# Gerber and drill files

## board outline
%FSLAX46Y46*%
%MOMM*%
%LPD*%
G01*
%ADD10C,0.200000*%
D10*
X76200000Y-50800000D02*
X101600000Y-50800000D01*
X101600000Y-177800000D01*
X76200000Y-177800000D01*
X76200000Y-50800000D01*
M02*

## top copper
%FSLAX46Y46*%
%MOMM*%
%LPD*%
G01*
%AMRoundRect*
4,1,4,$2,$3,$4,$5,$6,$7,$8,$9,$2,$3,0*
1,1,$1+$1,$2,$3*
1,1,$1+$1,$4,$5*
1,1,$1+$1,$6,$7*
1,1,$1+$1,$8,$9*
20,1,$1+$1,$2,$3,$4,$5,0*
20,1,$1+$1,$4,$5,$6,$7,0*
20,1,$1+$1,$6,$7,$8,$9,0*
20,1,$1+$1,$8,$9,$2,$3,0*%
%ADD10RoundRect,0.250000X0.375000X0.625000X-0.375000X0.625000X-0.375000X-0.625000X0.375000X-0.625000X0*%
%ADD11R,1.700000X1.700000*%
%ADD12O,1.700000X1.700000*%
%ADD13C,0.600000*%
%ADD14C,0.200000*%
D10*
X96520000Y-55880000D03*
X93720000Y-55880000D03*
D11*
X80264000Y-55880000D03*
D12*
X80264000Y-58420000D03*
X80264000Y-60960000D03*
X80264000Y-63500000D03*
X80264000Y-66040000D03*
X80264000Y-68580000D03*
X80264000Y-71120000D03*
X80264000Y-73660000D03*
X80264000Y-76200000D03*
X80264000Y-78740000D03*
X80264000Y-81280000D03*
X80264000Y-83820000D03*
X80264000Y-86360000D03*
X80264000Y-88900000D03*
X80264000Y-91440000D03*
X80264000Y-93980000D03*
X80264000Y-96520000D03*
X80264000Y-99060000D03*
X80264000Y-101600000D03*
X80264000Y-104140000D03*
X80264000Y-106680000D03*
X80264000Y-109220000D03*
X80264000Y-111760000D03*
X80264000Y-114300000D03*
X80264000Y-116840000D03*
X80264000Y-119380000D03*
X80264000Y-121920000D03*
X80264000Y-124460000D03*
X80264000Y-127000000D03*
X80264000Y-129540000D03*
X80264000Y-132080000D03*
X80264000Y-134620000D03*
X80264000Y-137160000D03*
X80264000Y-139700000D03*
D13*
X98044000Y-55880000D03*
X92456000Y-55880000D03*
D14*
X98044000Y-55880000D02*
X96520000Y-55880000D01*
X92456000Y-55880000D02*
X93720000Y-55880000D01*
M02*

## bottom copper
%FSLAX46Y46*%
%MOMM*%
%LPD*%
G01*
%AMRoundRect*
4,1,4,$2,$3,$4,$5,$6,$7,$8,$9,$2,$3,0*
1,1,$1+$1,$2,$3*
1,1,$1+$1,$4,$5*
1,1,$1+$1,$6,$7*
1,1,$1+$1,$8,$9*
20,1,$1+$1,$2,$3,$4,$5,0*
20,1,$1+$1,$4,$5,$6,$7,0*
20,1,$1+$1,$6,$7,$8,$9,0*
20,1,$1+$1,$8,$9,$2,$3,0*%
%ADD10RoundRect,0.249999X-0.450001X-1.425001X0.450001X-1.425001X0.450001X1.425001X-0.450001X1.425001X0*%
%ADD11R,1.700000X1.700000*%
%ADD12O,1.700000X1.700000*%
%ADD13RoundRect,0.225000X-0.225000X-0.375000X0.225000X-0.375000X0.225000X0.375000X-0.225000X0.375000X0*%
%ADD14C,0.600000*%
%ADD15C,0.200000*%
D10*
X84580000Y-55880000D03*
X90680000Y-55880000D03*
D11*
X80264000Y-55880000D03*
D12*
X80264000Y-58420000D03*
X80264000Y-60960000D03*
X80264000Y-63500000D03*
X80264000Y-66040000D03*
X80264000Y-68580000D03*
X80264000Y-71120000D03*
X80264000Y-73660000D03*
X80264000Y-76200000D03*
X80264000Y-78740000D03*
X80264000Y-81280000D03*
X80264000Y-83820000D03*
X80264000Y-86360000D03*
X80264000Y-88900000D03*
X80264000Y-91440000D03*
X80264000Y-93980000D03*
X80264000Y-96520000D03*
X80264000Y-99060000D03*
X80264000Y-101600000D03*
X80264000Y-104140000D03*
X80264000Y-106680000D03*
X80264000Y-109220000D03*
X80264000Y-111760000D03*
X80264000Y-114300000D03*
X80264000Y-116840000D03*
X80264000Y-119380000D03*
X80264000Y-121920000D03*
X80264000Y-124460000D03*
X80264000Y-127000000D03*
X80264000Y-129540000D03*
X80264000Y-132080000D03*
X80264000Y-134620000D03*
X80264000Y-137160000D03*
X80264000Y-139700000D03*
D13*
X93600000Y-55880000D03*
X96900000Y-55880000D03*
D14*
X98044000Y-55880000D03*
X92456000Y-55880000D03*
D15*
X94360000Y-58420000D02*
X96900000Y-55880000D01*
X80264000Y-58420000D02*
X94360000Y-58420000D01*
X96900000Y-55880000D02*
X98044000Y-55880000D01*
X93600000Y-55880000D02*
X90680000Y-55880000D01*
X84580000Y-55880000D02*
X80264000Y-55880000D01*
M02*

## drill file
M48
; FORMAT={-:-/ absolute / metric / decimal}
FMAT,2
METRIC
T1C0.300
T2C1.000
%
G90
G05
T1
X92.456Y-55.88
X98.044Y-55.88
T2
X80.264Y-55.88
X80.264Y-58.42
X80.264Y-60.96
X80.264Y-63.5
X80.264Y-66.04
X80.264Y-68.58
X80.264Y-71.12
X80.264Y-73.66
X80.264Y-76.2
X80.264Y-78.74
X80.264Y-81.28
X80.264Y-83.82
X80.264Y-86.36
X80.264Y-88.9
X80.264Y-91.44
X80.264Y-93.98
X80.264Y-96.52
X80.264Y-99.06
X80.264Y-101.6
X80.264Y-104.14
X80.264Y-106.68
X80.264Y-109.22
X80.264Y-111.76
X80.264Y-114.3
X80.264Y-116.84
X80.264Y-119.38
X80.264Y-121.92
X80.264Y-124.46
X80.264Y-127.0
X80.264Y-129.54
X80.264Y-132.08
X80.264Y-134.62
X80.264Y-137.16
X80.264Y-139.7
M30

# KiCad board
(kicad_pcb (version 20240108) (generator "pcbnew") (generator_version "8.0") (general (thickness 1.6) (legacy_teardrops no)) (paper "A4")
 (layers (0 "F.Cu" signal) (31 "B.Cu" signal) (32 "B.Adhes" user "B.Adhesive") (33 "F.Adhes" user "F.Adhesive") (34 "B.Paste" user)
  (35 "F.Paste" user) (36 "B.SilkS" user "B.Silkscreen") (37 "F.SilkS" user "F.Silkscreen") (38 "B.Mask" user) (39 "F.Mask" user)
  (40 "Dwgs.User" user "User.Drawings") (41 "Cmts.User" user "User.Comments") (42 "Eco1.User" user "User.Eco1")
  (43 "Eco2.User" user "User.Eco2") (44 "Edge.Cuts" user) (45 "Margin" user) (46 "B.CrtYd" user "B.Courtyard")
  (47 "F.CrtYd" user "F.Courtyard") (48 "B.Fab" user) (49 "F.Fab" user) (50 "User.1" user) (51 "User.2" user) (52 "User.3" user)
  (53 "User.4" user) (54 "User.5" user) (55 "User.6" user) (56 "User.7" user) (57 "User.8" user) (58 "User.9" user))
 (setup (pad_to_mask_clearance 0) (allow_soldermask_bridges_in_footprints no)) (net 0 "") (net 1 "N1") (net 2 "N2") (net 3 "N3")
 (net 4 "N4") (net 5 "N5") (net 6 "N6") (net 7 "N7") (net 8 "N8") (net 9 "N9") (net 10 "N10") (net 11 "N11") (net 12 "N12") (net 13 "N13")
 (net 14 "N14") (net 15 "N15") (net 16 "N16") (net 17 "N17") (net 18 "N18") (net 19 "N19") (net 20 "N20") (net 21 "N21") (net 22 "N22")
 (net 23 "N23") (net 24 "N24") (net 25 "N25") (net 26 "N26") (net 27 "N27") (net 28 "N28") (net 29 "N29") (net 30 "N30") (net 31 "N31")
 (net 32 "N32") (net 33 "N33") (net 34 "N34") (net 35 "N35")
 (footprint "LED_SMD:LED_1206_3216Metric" (layer "F.Cu") (at 95.12 55.88 180)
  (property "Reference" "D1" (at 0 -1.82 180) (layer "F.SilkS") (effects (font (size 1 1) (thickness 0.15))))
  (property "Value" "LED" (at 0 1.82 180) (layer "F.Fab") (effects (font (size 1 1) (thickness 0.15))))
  (pad "1" smd roundrect (at -1.4 0 180) (size 1.25 1.75) (layers "F.Cu" "F.Paste" "F.Mask") (roundrect_rratio 0.2) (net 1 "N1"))
  (pad "2" smd roundrect (at 1.4 0 180) (size 1.25 1.75) (layers "F.Cu" "F.Paste" "F.Mask") (roundrect_rratio 0.2) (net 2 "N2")))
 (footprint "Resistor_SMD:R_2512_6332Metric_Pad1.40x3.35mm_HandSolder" (layer "B.Cu") (at 87.63 55.88)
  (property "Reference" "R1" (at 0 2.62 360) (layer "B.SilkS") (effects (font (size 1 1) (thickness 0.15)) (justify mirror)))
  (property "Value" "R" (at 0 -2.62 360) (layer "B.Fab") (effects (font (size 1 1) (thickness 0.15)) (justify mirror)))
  (pad "1" smd roundrect (at -3.05 0) (size 1.4 3.35) (layers "B.Cu" "B.Paste" "B.Mask") (roundrect_rratio 0.178571) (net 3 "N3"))
  (pad "2" smd roundrect (at 3.05 0) (size 1.4 3.35) (layers "B.Cu" "B.Paste" "B.Mask") (roundrect_rratio 0.178571) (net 2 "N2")))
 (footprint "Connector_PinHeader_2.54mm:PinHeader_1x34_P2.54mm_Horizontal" (layer "B.Cu") (at 80.264 55.88 180)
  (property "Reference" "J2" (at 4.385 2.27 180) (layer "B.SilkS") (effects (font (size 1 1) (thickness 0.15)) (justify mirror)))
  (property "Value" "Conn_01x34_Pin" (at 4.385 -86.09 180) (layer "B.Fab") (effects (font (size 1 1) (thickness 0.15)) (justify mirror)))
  (pad "1" thru_hole rect (at 0 0 180) (size 1.7 1.7) (drill 1) (layers "*.Cu" "*.Mask") (remove_unused_layers no) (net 3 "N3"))
  (pad "2" thru_hole oval (at 0 -2.54 180) (size 1.7 1.7) (drill 1) (layers "*.Cu" "*.Mask") (remove_unused_layers no) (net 1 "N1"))
  (pad "3" thru_hole oval (at 0 -5.08 180) (size 1.7 1.7) (drill 1) (layers "*.Cu" "*.Mask") (remove_unused_layers no) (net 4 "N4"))
  (pad "4" thru_hole oval (at 0 -7.62 180) (size 1.7 1.7) (drill 1) (layers "*.Cu" "*.Mask") (remove_unused_layers no) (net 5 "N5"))
  (pad "5" thru_hole oval (at 0 -10.16 180) (size 1.7 1.7) (drill 1) (layers "*.Cu" "*.Mask") (remove_unused_layers no) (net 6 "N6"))
  (pad "6" thru_hole oval (at 0 -12.7 180) (size 1.7 1.7) (drill 1) (layers "*.Cu" "*.Mask") (remove_unused_layers no) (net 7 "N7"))
  (pad "7" thru_hole oval (at 0 -15.24 180) (size 1.7 1.7) (drill 1) (layers "*.Cu" "*.Mask") (remove_unused_layers no) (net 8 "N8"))
  (pad "8" thru_hole oval (at 0 -17.78 180) (size 1.7 1.7) (drill 1) (layers "*.Cu" "*.Mask") (remove_unused_layers no) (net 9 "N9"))
  (pad "9" thru_hole oval (at 0 -20.32 180) (size 1.7 1.7) (drill 1) (layers "*.Cu" "*.Mask") (remove_unused_layers no) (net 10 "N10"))
  (pad "10" thru_hole oval (at 0 -22.86 180) (size 1.7 1.7) (drill 1) (layers "*.Cu" "*.Mask") (remove_unused_layers no) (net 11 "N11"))
  (pad "11" thru_hole oval (at 0 -25.4 180) (size 1.7 1.7) (drill 1) (layers "*.Cu" "*.Mask") (remove_unused_layers no) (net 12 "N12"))
  (pad "12" thru_hole oval (at 0 -27.94 180) (size 1.7 1.7) (drill 1) (layers "*.Cu" "*.Mask") (remove_unused_layers no) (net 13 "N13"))
  (pad "13" thru_hole oval (at 0 -30.48 180) (size 1.7 1.7) (drill 1) (layers "*.Cu" "*.Mask") (remove_unused_layers no) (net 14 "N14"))
  (pad "14" thru_hole oval (at 0 -33.02 180) (size 1.7 1.7) (drill 1) (layers "*.Cu" "*.Mask") (remove_unused_layers no) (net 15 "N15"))
  (pad "15" thru_hole oval (at 0 -35.56 180) (size 1.7 1.7) (drill 1) (layers "*.Cu" "*.Mask") (remove_unused_layers no) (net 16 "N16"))
  (pad "16" thru_hole oval (at 0 -38.1 180) (size 1.7 1.7) (drill 1) (layers "*.Cu" "*.Mask") (remove_unused_layers no) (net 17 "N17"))
  (pad "17" thru_hole oval (at 0 -40.64 180) (size 1.7 1.7) (drill 1) (layers "*.Cu" "*.Mask") (remove_unused_layers no) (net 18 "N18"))
  (pad "18" thru_hole oval (at 0 -43.18 180) (size 1.7 1.7) (drill 1) (layers "*.Cu" "*.Mask") (remove_unused_layers no) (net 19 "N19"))
  (pad "19" thru_hole oval (at 0 -45.72 180) (size 1.7 1.7) (drill 1) (layers "*.Cu" "*.Mask") (remove_unused_layers no) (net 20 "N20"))
  (pad "20" thru_hole oval (at 0 -48.26 180) (size 1.7 1.7) (drill 1) (layers "*.Cu" "*.Mask") (remove_unused_layers no) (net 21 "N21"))
  (pad "21" thru_hole oval (at 0 -50.8 180) (size 1.7 1.7) (drill 1) (layers "*.Cu" "*.Mask") (remove_unused_layers no) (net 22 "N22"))
  (pad "22" thru_hole oval (at 0 -53.34 180) (size 1.7 1.7) (drill 1) (layers "*.Cu" "*.Mask") (remove_unused_layers no) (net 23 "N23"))
  (pad "23" thru_hole oval (at 0 -55.88 180) (size 1.7 1.7) (drill 1) (layers "*.Cu" "*.Mask") (remove_unused_layers no) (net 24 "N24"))
  (pad "24" thru_hole oval (at 0 -58.42 180) (size 1.7 1.7) (drill 1) (layers "*.Cu" "*.Mask") (remove_unused_layers no) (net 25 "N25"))
  (pad "25" thru_hole oval (at 0 -60.96 180) (size 1.7 1.7) (drill 1) (layers "*.Cu" "*.Mask") (remove_unused_layers no) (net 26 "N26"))
  (pad "26" thru_hole oval (at 0 -63.5 180) (size 1.7 1.7) (drill 1) (layers "*.Cu" "*.Mask") (remove_unused_layers no) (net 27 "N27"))
  (pad "27" thru_hole oval (at 0 -66.04 180) (size 1.7 1.7) (drill 1) (layers "*.Cu" "*.Mask") (remove_unused_layers no) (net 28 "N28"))
  (pad "28" thru_hole oval (at 0 -68.58 180) (size 1.7 1.7) (drill 1) (layers "*.Cu" "*.Mask") (remove_unused_layers no) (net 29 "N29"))
  (pad "29" thru_hole oval (at 0 -71.12 180) (size 1.7 1.7) (drill 1) (layers "*.Cu" "*.Mask") (remove_unused_layers no) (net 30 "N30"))
  (pad "30" thru_hole oval (at 0 -73.66 180) (size 1.7 1.7) (drill 1) (layers "*.Cu" "*.Mask") (remove_unused_layers no) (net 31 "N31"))
  (pad "31" thru_hole oval (at 0 -76.2 180) (size 1.7 1.7) (drill 1) (layers "*.Cu" "*.Mask") (remove_unused_layers no) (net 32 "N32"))
  (pad "32" thru_hole oval (at 0 -78.74 180) (size 1.7 1.7) (drill 1) (layers "*.Cu" "*.Mask") (remove_unused_layers no) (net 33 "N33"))
  (pad "33" thru_hole oval (at 0 -81.28 180) (size 1.7 1.7) (drill 1) (layers "*.Cu" "*.Mask") (remove_unused_layers no) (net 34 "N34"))
  (pad "34" thru_hole oval (at 0 -83.82 180) (size 1.7 1.7) (drill 1) (layers "*.Cu" "*.Mask") (remove_unused_layers no) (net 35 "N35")))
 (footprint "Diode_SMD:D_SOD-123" (layer "B.Cu") (at 95.25 55.88)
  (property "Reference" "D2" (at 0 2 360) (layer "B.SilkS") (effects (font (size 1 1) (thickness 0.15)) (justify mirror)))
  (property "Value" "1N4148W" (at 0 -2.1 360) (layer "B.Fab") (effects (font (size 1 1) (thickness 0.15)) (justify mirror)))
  (pad "1" smd roundrect (at -1.65 0) (size 0.9 1.2) (layers "B.Cu" "B.Paste" "B.Mask") (roundrect_rratio 0.25) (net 2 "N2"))
  (pad "2" smd roundrect (at 1.65 0) (size 0.9 1.2) (layers "B.Cu" "B.Paste" "B.Mask") (roundrect_rratio 0.25) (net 1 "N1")))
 (gr_rect (start 76.2 50.8) (end 101.6 177.8) (stroke (width 0.2) (type default)) (fill none) (layer "Edge.Cuts"))
 (segment (start 98.044 55.88) (end 96.52 55.88) (width 0.2) (layer "F.Cu") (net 1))
 (via (at 98.044 55.88) (size 0.6) (drill 0.3) (layers "F.Cu" "B.Cu") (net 1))
 (segment (start 94.36 58.42) (end 96.9 55.88) (width 0.2) (layer "B.Cu") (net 1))
 (segment (start 80.264 58.42) (end 94.36 58.42) (width 0.2) (layer "B.Cu") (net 1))
 (segment (start 96.9 55.88) (end 98.044 55.88) (width 0.2) (layer "B.Cu") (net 1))
 (segment (start 92.456 55.88) (end 93.72 55.88) (width 0.2) (layer "F.Cu") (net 2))
 (via (at 92.456 55.88) (size 0.6) (drill 0.3) (layers "F.Cu" "B.Cu") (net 2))
 (segment (start 93.6 55.88) (end 90.68 55.88) (width 0.2) (layer "B.Cu") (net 2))
 (segment (start 84.58 55.88) (end 80.264 55.88) (width 0.2) (layer "B.Cu") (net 3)))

